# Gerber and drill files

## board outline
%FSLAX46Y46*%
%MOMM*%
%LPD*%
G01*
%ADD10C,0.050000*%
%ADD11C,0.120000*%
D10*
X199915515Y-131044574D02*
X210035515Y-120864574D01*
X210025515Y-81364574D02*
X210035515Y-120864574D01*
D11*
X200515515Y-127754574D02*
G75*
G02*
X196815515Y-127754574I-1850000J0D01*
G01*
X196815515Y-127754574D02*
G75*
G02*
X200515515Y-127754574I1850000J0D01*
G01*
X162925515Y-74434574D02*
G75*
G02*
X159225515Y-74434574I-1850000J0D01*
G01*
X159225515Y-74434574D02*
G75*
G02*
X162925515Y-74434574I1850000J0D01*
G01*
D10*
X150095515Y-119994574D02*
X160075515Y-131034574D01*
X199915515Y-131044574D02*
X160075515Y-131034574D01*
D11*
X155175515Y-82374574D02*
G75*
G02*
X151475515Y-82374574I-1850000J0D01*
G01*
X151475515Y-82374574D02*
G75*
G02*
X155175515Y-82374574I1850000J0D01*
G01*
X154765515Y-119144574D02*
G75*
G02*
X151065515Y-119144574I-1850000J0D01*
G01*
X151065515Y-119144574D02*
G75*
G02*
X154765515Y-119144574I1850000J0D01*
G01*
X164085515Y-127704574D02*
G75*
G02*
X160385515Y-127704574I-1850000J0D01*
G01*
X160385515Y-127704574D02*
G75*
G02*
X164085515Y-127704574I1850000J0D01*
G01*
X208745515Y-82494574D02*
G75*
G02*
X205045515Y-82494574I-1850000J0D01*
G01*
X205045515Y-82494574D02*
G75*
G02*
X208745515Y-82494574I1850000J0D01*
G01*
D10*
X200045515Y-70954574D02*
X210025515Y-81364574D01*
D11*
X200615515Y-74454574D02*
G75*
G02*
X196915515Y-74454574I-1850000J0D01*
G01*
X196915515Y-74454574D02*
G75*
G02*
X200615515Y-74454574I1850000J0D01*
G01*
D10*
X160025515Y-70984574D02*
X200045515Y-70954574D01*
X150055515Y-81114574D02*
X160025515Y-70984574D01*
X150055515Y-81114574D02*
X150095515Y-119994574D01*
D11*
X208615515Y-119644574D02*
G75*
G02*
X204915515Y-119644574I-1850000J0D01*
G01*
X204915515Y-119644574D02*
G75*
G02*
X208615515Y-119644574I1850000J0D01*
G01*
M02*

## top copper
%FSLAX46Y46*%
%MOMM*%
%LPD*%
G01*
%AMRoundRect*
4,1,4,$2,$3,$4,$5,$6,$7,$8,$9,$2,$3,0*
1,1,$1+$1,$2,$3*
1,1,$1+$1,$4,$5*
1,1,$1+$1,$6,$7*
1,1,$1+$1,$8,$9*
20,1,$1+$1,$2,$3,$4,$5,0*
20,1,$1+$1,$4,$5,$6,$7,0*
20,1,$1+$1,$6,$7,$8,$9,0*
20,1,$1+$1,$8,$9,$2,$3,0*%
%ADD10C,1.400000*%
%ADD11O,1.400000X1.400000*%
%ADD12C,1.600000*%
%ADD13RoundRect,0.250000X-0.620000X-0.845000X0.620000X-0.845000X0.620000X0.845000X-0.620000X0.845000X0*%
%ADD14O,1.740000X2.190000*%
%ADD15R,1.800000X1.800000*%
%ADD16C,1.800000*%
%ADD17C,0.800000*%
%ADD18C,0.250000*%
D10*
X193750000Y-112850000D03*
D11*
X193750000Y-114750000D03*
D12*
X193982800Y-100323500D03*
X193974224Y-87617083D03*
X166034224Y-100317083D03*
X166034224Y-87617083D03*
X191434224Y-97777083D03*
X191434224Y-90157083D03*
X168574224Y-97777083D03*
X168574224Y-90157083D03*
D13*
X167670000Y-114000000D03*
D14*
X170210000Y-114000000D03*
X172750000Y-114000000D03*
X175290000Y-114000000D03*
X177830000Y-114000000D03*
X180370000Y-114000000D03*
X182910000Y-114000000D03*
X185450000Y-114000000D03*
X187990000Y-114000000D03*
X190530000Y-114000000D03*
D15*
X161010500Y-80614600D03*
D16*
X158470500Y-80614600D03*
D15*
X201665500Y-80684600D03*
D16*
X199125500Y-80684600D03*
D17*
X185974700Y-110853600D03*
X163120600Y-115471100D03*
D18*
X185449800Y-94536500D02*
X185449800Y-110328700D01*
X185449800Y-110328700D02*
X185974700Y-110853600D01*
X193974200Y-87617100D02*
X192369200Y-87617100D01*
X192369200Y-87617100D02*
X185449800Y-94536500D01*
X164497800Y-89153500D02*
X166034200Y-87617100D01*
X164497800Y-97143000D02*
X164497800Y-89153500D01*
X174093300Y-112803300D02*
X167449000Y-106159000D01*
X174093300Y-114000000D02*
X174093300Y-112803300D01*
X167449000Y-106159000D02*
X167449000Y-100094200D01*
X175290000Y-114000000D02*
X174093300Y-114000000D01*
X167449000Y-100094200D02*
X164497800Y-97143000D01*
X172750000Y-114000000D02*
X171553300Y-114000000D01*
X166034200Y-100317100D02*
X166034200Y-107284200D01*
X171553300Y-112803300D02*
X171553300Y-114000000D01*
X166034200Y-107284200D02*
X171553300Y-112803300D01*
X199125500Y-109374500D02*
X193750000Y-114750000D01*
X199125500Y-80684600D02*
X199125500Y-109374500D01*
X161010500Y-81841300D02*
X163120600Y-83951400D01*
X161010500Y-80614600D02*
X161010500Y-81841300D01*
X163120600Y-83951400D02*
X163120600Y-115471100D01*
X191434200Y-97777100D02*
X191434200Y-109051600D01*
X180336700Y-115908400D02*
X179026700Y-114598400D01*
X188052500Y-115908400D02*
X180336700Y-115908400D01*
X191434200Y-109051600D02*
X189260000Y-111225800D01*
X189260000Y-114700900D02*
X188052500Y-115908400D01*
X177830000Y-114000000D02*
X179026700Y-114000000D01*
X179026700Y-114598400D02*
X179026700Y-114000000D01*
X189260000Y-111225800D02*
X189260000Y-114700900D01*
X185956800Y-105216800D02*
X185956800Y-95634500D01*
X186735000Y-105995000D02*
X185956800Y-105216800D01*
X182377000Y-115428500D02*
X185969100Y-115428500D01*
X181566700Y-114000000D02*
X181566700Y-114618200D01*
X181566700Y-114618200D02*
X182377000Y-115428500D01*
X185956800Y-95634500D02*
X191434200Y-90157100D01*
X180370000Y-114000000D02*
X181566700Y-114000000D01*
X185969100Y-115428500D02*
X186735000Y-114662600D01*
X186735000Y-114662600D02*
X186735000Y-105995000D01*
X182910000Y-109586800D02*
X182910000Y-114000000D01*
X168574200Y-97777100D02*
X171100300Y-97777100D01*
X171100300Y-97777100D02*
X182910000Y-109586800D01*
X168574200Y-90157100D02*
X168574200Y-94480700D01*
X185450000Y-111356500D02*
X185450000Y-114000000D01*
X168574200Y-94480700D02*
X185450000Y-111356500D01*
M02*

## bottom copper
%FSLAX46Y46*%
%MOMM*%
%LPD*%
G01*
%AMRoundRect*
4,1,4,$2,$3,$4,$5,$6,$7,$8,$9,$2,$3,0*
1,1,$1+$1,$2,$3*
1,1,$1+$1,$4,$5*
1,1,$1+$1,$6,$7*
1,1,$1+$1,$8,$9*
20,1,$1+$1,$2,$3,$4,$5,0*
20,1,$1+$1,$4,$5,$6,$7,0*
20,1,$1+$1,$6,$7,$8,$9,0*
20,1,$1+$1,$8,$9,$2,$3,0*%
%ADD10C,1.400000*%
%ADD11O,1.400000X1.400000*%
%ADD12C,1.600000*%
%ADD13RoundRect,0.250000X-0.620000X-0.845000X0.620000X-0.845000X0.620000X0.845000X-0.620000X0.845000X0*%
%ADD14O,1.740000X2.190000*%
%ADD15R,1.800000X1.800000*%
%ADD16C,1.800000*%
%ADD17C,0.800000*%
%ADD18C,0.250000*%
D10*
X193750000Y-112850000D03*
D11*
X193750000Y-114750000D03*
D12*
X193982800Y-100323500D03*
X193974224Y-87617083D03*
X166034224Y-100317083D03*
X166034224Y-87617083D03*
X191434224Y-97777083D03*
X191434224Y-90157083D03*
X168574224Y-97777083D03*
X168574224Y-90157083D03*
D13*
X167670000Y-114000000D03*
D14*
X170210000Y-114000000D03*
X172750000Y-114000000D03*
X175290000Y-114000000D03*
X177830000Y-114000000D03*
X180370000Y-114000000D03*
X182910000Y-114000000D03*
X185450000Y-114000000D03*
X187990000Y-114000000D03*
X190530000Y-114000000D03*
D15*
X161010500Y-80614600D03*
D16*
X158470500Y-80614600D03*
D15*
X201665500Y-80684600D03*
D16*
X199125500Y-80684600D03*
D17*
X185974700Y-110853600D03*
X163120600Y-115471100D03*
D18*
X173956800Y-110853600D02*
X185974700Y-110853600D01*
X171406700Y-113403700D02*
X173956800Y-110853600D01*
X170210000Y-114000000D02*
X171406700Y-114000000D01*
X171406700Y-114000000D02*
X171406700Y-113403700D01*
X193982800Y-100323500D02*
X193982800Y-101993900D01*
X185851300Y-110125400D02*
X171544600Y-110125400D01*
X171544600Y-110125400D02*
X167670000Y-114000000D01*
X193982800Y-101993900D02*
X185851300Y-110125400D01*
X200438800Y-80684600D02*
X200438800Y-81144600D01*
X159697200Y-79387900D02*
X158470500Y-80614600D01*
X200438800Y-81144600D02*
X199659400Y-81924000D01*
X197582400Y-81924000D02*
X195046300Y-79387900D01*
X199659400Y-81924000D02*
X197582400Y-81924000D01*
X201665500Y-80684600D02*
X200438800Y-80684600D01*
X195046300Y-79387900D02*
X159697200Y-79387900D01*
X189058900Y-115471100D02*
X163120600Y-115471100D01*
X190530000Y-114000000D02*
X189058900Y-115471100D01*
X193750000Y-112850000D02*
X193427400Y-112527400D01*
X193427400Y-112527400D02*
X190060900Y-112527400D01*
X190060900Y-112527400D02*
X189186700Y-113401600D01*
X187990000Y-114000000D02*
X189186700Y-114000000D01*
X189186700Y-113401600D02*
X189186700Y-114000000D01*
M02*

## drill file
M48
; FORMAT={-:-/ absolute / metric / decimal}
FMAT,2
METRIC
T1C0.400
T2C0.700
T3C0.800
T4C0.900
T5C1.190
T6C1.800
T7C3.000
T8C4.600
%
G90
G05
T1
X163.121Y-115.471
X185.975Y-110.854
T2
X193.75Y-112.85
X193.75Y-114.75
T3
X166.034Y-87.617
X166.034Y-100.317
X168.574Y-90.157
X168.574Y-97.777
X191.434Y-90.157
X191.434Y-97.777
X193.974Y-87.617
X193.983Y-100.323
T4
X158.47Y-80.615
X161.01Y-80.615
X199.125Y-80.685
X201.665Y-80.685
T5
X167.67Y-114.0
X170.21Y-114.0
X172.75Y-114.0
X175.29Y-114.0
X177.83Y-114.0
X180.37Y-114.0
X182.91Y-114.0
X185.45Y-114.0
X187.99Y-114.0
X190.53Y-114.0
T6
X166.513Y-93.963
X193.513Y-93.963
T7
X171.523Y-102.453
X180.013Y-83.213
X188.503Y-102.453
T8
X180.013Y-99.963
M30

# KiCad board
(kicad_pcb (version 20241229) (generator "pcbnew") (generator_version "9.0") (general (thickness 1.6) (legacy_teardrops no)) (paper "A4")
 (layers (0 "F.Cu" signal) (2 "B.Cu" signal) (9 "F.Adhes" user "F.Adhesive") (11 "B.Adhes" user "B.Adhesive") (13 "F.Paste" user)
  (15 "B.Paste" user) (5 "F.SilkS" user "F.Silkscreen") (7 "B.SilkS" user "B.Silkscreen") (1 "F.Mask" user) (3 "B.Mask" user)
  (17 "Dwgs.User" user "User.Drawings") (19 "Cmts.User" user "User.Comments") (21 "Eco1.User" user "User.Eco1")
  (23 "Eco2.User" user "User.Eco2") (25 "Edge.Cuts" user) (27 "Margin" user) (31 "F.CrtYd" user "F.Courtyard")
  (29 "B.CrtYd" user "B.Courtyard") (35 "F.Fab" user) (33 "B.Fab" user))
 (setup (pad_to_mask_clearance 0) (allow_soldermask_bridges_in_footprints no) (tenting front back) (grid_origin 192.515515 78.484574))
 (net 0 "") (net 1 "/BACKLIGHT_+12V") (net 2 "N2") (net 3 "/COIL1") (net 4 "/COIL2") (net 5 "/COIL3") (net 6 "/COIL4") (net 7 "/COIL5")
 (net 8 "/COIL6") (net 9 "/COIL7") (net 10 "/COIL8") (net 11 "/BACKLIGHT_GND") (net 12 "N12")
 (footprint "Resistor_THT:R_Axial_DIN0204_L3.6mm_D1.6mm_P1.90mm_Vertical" (layer "F.Cu") (at 193.75 112.85 -90)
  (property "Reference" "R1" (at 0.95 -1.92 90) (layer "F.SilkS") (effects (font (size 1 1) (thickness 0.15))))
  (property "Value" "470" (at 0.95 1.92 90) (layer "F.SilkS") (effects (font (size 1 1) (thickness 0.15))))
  (pad "1" thru_hole circle (at 0 0 270) (size 1.4 1.4) (drill 0.7) (layers "*.Cu" "*.Mask") (remove_unused_layers no)
   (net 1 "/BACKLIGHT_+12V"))
  (pad "2" thru_hole oval (at 1.9 0 270) (size 1.4 1.4) (drill 0.7) (layers "*.Cu" "*.Mask") (remove_unused_layers no) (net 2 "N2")))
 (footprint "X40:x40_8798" (layer "F.Cu") (at 180.0128 93.9635 180)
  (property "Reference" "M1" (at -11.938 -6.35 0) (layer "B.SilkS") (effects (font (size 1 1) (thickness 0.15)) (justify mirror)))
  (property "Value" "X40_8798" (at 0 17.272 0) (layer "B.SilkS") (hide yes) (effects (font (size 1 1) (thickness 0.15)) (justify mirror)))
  (pad "" np_thru_hole circle (at -13.5 0 180) (size 1.8 1.8) (drill 1.8) (layers "*.Cu" "*.Mask"))
  (pad "" np_thru_hole circle (at -8.49 -8.49 180) (size 3 3) (drill 3) (layers "*.Cu" "*.Mask"))
  (pad "" np_thru_hole circle (at 0 -6 180) (size 4.6 4.6) (drill 4.6) (layers "*.Cu" "*.Mask"))
  (pad "" np_thru_hole circle (at 0 10.75 180) (size 3 3) (drill 3) (layers "*.Cu" "*.Mask"))
  (pad "" np_thru_hole circle (at 8.49 -8.49 180) (size 3 3) (drill 3) (layers "*.Cu" "*.Mask"))
  (pad "" np_thru_hole circle (at 13.5 0 180) (size 1.8 1.8) (drill 1.8) (layers "*.Cu" "*.Mask"))
  (pad "1" thru_hole circle (at -13.97 -6.36 180) (size 1.6 1.6) (drill 0.8) (layers "*.Cu" "*.Mask") (remove_unused_layers no)
   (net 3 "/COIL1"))
  (pad "2" thru_hole circle (at -13.961424 6.346417 180) (size 1.6 1.6) (drill 0.8) (layers "*.Cu" "*.Mask") (remove_unused_layers no)
   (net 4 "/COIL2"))
  (pad "3" thru_hole circle (at 13.978576 -6.353583 180) (size 1.6 1.6) (drill 0.8) (layers "*.Cu" "*.Mask") (remove_unused_layers no)
   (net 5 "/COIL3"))
  (pad "4" thru_hole circle (at 13.978576 6.346417 180) (size 1.6 1.6) (drill 0.8) (layers "*.Cu" "*.Mask") (remove_unused_layers no)
   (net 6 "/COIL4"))
  (pad "5" thru_hole circle (at -11.421424 -3.813583 180) (size 1.6 1.6) (drill 0.8) (layers "*.Cu" "*.Mask") (remove_unused_layers no)
   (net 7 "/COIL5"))
  (pad "6" thru_hole circle (at -11.421424 3.806417 180) (size 1.6 1.6) (drill 0.8) (layers "*.Cu" "*.Mask") (remove_unused_layers no)
   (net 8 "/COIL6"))
  (pad "7" thru_hole circle (at 11.438576 -3.813583 180) (size 1.6 1.6) (drill 0.8) (layers "*.Cu" "*.Mask") (remove_unused_layers no)
   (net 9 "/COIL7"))
  (pad "8" thru_hole circle (at 11.438576 3.806417 180) (size 1.6 1.6) (drill 0.8) (layers "*.Cu" "*.Mask") (remove_unused_layers no)
   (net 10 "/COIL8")))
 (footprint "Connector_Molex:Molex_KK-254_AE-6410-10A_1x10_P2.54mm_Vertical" (layer "F.Cu") (at 167.67 114)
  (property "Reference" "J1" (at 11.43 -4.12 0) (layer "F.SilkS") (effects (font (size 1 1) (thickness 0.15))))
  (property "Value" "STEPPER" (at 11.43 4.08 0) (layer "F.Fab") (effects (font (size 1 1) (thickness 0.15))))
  (pad "1" thru_hole roundrect (at 0 0) (size 1.74 2.19) (drill 1.19) (layers "*.Cu" "*.Mask") (remove_unused_layers no)
   (roundrect_rratio 0.143678) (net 3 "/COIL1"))
  (pad "2" thru_hole oval (at 2.54 0) (size 1.74 2.19) (drill 1.19) (layers "*.Cu" "*.Mask") (remove_unused_layers no) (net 4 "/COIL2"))
  (pad "3" thru_hole oval (at 5.08 0) (size 1.74 2.19) (drill 1.19) (layers "*.Cu" "*.Mask") (remove_unused_layers no) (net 5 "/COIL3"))
  (pad "4" thru_hole oval (at 7.62 0) (size 1.74 2.19) (drill 1.19) (layers "*.Cu" "*.Mask") (remove_unused_layers no) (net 6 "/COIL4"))
  (pad "5" thru_hole oval (at 10.16 0) (size 1.74 2.19) (drill 1.19) (layers "*.Cu" "*.Mask") (remove_unused_layers no) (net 7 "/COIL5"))
  (pad "6" thru_hole oval (at 12.7 0) (size 1.74 2.19) (drill 1.19) (layers "*.Cu" "*.Mask") (remove_unused_layers no) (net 8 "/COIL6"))
  (pad "7" thru_hole oval (at 15.24 0) (size 1.74 2.19) (drill 1.19) (layers "*.Cu" "*.Mask") (remove_unused_layers no) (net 9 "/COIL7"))
  (pad "8" thru_hole oval (at 17.78 0) (size 1.74 2.19) (drill 1.19) (layers "*.Cu" "*.Mask") (remove_unused_layers no) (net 10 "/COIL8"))
  (pad "9" thru_hole oval (at 20.32 0) (size 1.74 2.19) (drill 1.19) (layers "*.Cu" "*.Mask") (remove_unused_layers no)
   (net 1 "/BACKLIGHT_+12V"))
  (pad "10" thru_hole oval (at 22.86 0) (size 1.74 2.19) (drill 1.19) (layers "*.Cu" "*.Mask") (remove_unused_layers no)
   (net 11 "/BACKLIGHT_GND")))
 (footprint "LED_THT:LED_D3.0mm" (layer "B.Cu") (at 161.0105 80.6146 180)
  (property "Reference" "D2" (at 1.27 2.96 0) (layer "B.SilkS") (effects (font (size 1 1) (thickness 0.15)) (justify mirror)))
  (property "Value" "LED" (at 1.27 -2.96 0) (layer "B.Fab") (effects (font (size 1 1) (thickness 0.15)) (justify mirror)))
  (pad "1" thru_hole rect (at 0 0 180) (size 1.8 1.8) (drill 0.9) (layers "*.Cu" "*.Mask") (remove_unused_layers no)
   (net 11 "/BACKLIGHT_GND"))
  (pad "2" thru_hole circle (at 2.54 0 180) (size 1.8 1.8) (drill 0.9) (layers "*.Cu" "*.Mask") (remove_unused_layers no) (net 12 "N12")))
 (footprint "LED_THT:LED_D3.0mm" (layer "B.Cu") (at 201.6655 80.6846 180)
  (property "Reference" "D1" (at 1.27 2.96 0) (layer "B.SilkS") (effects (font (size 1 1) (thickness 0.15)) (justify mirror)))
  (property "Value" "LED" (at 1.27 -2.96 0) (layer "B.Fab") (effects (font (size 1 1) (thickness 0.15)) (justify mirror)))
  (pad "1" thru_hole rect (at 0 0 180) (size 1.8 1.8) (drill 0.9) (layers "*.Cu" "*.Mask") (remove_unused_layers no) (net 12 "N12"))
  (pad "2" thru_hole circle (at 2.54 0 180) (size 1.8 1.8) (drill 0.9) (layers "*.Cu" "*.Mask") (remove_unused_layers no) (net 2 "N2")))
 (gr_line (start 199.915515 131.044574) (end 210.035515 120.864574) (stroke (width 0.05) (type solid)) (layer "Edge.Cuts"))
 (gr_line (start 210.025515 81.364574) (end 210.035515 120.864574) (stroke (width 0.05) (type solid)) (layer "Edge.Cuts"))
 (gr_circle (center 198.665515 127.754574) (end 200.515515 127.754574) (stroke (width 0.12) (type solid)) (fill no) (layer "Edge.Cuts"))
 (gr_circle (center 161.075515 74.434574) (end 162.925515 74.434574) (stroke (width 0.12) (type solid)) (fill no) (layer "Edge.Cuts"))
 (gr_line (start 150.095515 119.994574) (end 160.075515 131.034574) (stroke (width 0.05) (type solid)) (layer "Edge.Cuts"))
 (gr_line (start 199.915515 131.044574) (end 160.075515 131.034574) (stroke (width 0.05) (type solid)) (layer "Edge.Cuts"))
 (gr_circle (center 153.325515 82.374574) (end 155.175515 82.374574) (stroke (width 0.12) (type solid)) (fill no) (layer "Edge.Cuts"))
 (gr_circle (center 152.915515 119.144574) (end 154.765515 119.144574) (stroke (width 0.12) (type solid)) (fill no) (layer "Edge.Cuts"))
 (gr_circle (center 162.235515 127.704574) (end 164.085515 127.704574) (stroke (width 0.12) (type solid)) (fill no) (layer "Edge.Cuts"))
 (gr_circle (center 206.895515 82.494574) (end 208.745515 82.494574) (stroke (width 0.12) (type solid)) (fill no) (layer "Edge.Cuts"))
 (gr_line (start 200.045515 70.954574) (end 210.025515 81.364574) (stroke (width 0.05) (type solid)) (layer "Edge.Cuts"))
 (gr_circle (center 198.765515 74.454574) (end 200.615515 74.454574) (stroke (width 0.12) (type solid)) (fill no) (layer "Edge.Cuts"))
 (gr_line (start 160.025515 70.984574) (end 200.045515 70.954574) (stroke (width 0.05) (type solid)) (layer "Edge.Cuts"))
 (gr_line (start 150.055515 81.114574) (end 160.025515 70.984574) (stroke (width 0.05) (type solid)) (layer "Edge.Cuts"))
 (gr_line (start 150.055515 81.114574) (end 150.095515 119.994574) (stroke (width 0.05) (type solid)) (layer "Edge.Cuts"))
 (gr_circle (center 206.765515 119.644574) (end 208.615515 119.644574) (stroke (width 0.12) (type solid)) (fill no) (layer "Edge.Cuts"))
 (segment (start 185.4498 94.5365) (end 185.4498 110.3287) (width 0.25) (layer "F.Cu") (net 4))
 (segment (start 185.4498 110.3287) (end 185.9747 110.8536) (width 0.25) (layer "F.Cu") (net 4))
 (segment (start 193.9742 87.6171) (end 192.3692 87.6171) (width 0.25) (layer "F.Cu") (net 4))
 (segment (start 192.3692 87.6171) (end 185.4498 94.5365) (width 0.25) (layer "F.Cu") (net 4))
 (via (at 185.9747 110.8536) (size 0.8) (drill 0.4) (layers "F.Cu" "B.Cu") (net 4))
 (segment (start 173.9568 110.8536) (end 185.9747 110.8536) (width 0.25) (layer "B.Cu") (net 4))
 (segment (start 171.4067 113.4037) (end 173.9568 110.8536) (width 0.25) (layer "B.Cu") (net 4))
 (segment (start 170.21 114) (end 171.4067 114) (width 0.25) (layer "B.Cu") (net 4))
 (segment (start 171.4067 114) (end 171.4067 113.4037) (width 0.25) (layer "B.Cu") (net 4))
 (segment (start 193.9828 100.3235) (end 193.9828 101.9939) (width 0.25) (layer "B.Cu") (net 3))
 (segment (start 185.8513 110.1254) (end 171.5446 110.1254) (width 0.25) (layer "B.Cu") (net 3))
 (segment (start 171.5446 110.1254) (end 167.67 114) (width 0.25) (layer "B.Cu") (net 3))
 (segment (start 193.9828 101.9939) (end 185.8513 110.1254) (width 0.25) (layer "B.Cu") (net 3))
 (segment (start 164.4978 89.1535) (end 166.0342 87.6171) (width 0.25) (layer "F.Cu") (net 6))
 (segment (start 164.4978 97.143) (end 164.4978 89.1535) (width 0.25) (layer "F.Cu") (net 6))
 (segment (start 174.0933 112.8033) (end 167.449 106.159) (width 0.25) (layer "F.Cu") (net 6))
 (segment (start 174.0933 114) (end 174.0933 112.8033) (width 0.25) (layer "F.Cu") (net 6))
 (segment (start 167.449 106.159) (end 167.449 100.0942) (width 0.25) (layer "F.Cu") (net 6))
 (segment (start 175.29 114) (end 174.0933 114) (width 0.25) (layer "F.Cu") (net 6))
 (segment (start 167.449 100.0942) (end 164.4978 97.143) (width 0.25) (layer "F.Cu") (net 6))
 (segment (start 172.75 114) (end 171.5533 114) (width 0.25) (layer "F.Cu") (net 5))
 (segment (start 166.0342 100.3171) (end 166.0342 107.2842) (width 0.25) (layer "F.Cu") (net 5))
 (segment (start 171.5533 112.8033) (end 171.5533 114) (width 0.25) (layer "F.Cu") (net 5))
 (segment (start 166.0342 107.2842) (end 171.5533 112.8033) (width 0.25) (layer "F.Cu") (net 5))
 (segment (start 199.1255 109.3745) (end 193.75 114.75) (width 0.25) (layer "F.Cu") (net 2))
 (segment (start 199.1255 80.6846) (end 199.1255 109.3745) (width 0.25) (layer "F.Cu") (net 2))
 (segment (start 200.4388 80.6846) (end 200.4388 81.1446) (width 0.25) (layer "B.Cu") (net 12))
 (segment (start 159.6972 79.3879) (end 158.4705 80.6146) (width 0.25) (layer "B.Cu") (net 12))
 (segment (start 200.4388 81.1446) (end 199.6594 81.924) (width 0.25) (layer "B.Cu") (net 12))
 (segment (start 197.5824 81.924) (end 195.0463 79.3879) (width 0.25) (layer "B.Cu") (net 12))
 (segment (start 199.6594 81.924) (end 197.5824 81.924) (width 0.25) (layer "B.Cu") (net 12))
 (segment (start 201.6655 80.6846) (end 200.4388 80.6846) (width 0.25) (layer "B.Cu") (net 12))
 (segment (start 195.0463 79.3879) (end 159.6972 79.3879) (width 0.25) (layer "B.Cu") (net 12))
 (segment (start 161.0105 81.8413) (end 163.1206 83.9514) (width 0.25) (layer "F.Cu") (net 11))
 (segment (start 161.0105 80.6146) (end 161.0105 81.8413) (width 0.25) (layer "F.Cu") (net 11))
 (segment (start 163.1206 83.9514) (end 163.1206 115.4711) (width 0.25) (layer "F.Cu") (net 11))
 (via (at 163.1206 115.4711) (size 0.8) (drill 0.4) (layers "F.Cu" "B.Cu") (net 11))
 (segment (start 189.0589 115.4711) (end 163.1206 115.4711) (width 0.25) (layer "B.Cu") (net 11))
 (segment (start 190.53 114) (end 189.0589 115.4711) (width 0.25) (layer "B.Cu") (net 11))
 (segment (start 193.75 112.85) (end 193.4274 112.5274) (width 0.25) (layer "B.Cu") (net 1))
 (segment (start 193.4274 112.5274) (end 190.0609 112.5274) (width 0.25) (layer "B.Cu") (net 1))
 (segment (start 190.0609 112.5274) (end 189.1867 113.4016) (width 0.25) (layer "B.Cu") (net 1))
 (segment (start 187.99 114) (end 189.1867 114) (width 0.25) (layer "B.Cu") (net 1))
 (segment (start 189.1867 113.4016) (end 189.1867 114) (width 0.25) (layer "B.Cu") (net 1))
 (segment (start 191.4342 97.7771) (end 191.4342 109.0516) (width 0.25) (layer "F.Cu") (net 7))
 (segment (start 180.3367 115.9084) (end 179.0267 114.5984) (width 0.25) (layer "F.Cu") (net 7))
 (segment (start 188.0525 115.9084) (end 180.3367 115.9084) (width 0.25) (layer "F.Cu") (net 7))
 (segment (start 191.4342 109.0516) (end 189.26 111.2258) (width 0.25) (layer "F.Cu") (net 7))
 (segment (start 189.26 114.7009) (end 188.0525 115.9084) (width 0.25) (layer "F.Cu") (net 7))
 (segment (start 177.83 114) (end 179.0267 114) (width 0.25) (layer "F.Cu") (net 7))
 (segment (start 179.0267 114.5984) (end 179.0267 114) (width 0.25) (layer "F.Cu") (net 7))
 (segment (start 189.26 111.2258) (end 189.26 114.7009) (width 0.25) (layer "F.Cu") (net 7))
 (segment (start 185.9568 105.2168) (end 185.9568 95.6345) (width 0.25) (layer "F.Cu") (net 8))
 (segment (start 186.735 105.995) (end 185.9568 105.2168) (width 0.25) (layer "F.Cu") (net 8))
 (segment (start 182.377 115.4285) (end 185.9691 115.4285) (width 0.25) (layer "F.Cu") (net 8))
 (segment (start 181.5667 114) (end 181.5667 114.6182) (width 0.25) (layer "F.Cu") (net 8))
 (segment (start 181.5667 114.6182) (end 182.377 115.4285) (width 0.25) (layer "F.Cu") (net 8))
 (segment (start 185.9568 95.6345) (end 191.4342 90.1571) (width 0.25) (layer "F.Cu") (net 8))
 (segment (start 180.37 114) (end 181.5667 114) (width 0.25) (layer "F.Cu") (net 8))
 (segment (start 185.9691 115.4285) (end 186.735 114.6626) (width 0.25) (layer "F.Cu") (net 8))
 (segment (start 186.735 114.6626) (end 186.735 105.995) (width 0.25) (layer "F.Cu") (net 8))
 (segment (start 182.91 109.5868) (end 182.91 114) (width 0.25) (layer "F.Cu") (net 9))
 (segment (start 168.5742 97.7771) (end 171.1003 97.7771) (width 0.25) (layer "F.Cu") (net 9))
 (segment (start 171.1003 97.7771) (end 182.91 109.5868) (width 0.25) (layer "F.Cu") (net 9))
 (segment (start 168.5742 90.1571) (end 168.5742 94.4807) (width 0.25) (layer "F.Cu") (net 10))
 (segment (start 185.45 111.3565) (end 185.45 114) (width 0.25) (layer "F.Cu") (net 10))
 (segment (start 168.5742 94.4807) (end 185.45 111.3565) (width 0.25) (layer "F.Cu") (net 10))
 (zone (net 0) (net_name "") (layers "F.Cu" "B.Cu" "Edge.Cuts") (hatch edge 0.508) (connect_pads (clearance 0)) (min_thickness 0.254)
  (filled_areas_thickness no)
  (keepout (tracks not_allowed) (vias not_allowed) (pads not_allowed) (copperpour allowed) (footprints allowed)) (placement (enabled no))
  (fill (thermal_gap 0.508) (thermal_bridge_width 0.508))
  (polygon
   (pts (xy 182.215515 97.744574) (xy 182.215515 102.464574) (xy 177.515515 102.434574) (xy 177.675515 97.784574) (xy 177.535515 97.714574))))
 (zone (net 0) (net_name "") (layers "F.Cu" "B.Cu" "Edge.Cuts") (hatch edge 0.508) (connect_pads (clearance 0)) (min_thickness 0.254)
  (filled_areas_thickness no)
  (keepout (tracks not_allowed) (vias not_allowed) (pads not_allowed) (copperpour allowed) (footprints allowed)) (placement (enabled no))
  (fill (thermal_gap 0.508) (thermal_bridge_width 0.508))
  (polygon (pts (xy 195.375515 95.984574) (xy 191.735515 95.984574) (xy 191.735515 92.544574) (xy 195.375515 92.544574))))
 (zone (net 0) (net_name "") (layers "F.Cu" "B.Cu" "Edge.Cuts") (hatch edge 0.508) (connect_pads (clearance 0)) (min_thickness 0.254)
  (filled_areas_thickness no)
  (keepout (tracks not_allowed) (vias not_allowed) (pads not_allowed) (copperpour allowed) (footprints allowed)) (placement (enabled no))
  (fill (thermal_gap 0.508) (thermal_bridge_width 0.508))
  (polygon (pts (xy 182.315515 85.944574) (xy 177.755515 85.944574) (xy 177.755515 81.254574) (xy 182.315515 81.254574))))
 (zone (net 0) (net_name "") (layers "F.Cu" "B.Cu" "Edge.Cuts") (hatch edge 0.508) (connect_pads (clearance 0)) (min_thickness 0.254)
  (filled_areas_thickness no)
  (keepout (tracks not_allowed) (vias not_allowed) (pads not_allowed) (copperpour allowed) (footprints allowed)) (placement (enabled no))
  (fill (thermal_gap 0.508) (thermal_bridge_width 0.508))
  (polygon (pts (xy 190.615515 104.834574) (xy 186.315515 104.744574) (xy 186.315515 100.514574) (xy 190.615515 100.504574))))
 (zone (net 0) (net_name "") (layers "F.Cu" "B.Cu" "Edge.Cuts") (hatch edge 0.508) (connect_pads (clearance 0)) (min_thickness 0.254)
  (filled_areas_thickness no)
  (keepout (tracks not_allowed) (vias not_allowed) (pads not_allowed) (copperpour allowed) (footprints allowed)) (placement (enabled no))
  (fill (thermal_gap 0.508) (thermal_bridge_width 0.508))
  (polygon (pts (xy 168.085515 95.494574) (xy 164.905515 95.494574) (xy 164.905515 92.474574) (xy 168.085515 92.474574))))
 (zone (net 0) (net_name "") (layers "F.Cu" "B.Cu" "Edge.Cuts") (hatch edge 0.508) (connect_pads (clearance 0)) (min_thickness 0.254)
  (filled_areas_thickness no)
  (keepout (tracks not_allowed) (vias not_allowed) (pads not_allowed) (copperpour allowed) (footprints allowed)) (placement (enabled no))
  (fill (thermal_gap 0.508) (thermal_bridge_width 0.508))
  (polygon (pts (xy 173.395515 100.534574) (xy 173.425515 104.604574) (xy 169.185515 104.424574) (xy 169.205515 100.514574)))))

